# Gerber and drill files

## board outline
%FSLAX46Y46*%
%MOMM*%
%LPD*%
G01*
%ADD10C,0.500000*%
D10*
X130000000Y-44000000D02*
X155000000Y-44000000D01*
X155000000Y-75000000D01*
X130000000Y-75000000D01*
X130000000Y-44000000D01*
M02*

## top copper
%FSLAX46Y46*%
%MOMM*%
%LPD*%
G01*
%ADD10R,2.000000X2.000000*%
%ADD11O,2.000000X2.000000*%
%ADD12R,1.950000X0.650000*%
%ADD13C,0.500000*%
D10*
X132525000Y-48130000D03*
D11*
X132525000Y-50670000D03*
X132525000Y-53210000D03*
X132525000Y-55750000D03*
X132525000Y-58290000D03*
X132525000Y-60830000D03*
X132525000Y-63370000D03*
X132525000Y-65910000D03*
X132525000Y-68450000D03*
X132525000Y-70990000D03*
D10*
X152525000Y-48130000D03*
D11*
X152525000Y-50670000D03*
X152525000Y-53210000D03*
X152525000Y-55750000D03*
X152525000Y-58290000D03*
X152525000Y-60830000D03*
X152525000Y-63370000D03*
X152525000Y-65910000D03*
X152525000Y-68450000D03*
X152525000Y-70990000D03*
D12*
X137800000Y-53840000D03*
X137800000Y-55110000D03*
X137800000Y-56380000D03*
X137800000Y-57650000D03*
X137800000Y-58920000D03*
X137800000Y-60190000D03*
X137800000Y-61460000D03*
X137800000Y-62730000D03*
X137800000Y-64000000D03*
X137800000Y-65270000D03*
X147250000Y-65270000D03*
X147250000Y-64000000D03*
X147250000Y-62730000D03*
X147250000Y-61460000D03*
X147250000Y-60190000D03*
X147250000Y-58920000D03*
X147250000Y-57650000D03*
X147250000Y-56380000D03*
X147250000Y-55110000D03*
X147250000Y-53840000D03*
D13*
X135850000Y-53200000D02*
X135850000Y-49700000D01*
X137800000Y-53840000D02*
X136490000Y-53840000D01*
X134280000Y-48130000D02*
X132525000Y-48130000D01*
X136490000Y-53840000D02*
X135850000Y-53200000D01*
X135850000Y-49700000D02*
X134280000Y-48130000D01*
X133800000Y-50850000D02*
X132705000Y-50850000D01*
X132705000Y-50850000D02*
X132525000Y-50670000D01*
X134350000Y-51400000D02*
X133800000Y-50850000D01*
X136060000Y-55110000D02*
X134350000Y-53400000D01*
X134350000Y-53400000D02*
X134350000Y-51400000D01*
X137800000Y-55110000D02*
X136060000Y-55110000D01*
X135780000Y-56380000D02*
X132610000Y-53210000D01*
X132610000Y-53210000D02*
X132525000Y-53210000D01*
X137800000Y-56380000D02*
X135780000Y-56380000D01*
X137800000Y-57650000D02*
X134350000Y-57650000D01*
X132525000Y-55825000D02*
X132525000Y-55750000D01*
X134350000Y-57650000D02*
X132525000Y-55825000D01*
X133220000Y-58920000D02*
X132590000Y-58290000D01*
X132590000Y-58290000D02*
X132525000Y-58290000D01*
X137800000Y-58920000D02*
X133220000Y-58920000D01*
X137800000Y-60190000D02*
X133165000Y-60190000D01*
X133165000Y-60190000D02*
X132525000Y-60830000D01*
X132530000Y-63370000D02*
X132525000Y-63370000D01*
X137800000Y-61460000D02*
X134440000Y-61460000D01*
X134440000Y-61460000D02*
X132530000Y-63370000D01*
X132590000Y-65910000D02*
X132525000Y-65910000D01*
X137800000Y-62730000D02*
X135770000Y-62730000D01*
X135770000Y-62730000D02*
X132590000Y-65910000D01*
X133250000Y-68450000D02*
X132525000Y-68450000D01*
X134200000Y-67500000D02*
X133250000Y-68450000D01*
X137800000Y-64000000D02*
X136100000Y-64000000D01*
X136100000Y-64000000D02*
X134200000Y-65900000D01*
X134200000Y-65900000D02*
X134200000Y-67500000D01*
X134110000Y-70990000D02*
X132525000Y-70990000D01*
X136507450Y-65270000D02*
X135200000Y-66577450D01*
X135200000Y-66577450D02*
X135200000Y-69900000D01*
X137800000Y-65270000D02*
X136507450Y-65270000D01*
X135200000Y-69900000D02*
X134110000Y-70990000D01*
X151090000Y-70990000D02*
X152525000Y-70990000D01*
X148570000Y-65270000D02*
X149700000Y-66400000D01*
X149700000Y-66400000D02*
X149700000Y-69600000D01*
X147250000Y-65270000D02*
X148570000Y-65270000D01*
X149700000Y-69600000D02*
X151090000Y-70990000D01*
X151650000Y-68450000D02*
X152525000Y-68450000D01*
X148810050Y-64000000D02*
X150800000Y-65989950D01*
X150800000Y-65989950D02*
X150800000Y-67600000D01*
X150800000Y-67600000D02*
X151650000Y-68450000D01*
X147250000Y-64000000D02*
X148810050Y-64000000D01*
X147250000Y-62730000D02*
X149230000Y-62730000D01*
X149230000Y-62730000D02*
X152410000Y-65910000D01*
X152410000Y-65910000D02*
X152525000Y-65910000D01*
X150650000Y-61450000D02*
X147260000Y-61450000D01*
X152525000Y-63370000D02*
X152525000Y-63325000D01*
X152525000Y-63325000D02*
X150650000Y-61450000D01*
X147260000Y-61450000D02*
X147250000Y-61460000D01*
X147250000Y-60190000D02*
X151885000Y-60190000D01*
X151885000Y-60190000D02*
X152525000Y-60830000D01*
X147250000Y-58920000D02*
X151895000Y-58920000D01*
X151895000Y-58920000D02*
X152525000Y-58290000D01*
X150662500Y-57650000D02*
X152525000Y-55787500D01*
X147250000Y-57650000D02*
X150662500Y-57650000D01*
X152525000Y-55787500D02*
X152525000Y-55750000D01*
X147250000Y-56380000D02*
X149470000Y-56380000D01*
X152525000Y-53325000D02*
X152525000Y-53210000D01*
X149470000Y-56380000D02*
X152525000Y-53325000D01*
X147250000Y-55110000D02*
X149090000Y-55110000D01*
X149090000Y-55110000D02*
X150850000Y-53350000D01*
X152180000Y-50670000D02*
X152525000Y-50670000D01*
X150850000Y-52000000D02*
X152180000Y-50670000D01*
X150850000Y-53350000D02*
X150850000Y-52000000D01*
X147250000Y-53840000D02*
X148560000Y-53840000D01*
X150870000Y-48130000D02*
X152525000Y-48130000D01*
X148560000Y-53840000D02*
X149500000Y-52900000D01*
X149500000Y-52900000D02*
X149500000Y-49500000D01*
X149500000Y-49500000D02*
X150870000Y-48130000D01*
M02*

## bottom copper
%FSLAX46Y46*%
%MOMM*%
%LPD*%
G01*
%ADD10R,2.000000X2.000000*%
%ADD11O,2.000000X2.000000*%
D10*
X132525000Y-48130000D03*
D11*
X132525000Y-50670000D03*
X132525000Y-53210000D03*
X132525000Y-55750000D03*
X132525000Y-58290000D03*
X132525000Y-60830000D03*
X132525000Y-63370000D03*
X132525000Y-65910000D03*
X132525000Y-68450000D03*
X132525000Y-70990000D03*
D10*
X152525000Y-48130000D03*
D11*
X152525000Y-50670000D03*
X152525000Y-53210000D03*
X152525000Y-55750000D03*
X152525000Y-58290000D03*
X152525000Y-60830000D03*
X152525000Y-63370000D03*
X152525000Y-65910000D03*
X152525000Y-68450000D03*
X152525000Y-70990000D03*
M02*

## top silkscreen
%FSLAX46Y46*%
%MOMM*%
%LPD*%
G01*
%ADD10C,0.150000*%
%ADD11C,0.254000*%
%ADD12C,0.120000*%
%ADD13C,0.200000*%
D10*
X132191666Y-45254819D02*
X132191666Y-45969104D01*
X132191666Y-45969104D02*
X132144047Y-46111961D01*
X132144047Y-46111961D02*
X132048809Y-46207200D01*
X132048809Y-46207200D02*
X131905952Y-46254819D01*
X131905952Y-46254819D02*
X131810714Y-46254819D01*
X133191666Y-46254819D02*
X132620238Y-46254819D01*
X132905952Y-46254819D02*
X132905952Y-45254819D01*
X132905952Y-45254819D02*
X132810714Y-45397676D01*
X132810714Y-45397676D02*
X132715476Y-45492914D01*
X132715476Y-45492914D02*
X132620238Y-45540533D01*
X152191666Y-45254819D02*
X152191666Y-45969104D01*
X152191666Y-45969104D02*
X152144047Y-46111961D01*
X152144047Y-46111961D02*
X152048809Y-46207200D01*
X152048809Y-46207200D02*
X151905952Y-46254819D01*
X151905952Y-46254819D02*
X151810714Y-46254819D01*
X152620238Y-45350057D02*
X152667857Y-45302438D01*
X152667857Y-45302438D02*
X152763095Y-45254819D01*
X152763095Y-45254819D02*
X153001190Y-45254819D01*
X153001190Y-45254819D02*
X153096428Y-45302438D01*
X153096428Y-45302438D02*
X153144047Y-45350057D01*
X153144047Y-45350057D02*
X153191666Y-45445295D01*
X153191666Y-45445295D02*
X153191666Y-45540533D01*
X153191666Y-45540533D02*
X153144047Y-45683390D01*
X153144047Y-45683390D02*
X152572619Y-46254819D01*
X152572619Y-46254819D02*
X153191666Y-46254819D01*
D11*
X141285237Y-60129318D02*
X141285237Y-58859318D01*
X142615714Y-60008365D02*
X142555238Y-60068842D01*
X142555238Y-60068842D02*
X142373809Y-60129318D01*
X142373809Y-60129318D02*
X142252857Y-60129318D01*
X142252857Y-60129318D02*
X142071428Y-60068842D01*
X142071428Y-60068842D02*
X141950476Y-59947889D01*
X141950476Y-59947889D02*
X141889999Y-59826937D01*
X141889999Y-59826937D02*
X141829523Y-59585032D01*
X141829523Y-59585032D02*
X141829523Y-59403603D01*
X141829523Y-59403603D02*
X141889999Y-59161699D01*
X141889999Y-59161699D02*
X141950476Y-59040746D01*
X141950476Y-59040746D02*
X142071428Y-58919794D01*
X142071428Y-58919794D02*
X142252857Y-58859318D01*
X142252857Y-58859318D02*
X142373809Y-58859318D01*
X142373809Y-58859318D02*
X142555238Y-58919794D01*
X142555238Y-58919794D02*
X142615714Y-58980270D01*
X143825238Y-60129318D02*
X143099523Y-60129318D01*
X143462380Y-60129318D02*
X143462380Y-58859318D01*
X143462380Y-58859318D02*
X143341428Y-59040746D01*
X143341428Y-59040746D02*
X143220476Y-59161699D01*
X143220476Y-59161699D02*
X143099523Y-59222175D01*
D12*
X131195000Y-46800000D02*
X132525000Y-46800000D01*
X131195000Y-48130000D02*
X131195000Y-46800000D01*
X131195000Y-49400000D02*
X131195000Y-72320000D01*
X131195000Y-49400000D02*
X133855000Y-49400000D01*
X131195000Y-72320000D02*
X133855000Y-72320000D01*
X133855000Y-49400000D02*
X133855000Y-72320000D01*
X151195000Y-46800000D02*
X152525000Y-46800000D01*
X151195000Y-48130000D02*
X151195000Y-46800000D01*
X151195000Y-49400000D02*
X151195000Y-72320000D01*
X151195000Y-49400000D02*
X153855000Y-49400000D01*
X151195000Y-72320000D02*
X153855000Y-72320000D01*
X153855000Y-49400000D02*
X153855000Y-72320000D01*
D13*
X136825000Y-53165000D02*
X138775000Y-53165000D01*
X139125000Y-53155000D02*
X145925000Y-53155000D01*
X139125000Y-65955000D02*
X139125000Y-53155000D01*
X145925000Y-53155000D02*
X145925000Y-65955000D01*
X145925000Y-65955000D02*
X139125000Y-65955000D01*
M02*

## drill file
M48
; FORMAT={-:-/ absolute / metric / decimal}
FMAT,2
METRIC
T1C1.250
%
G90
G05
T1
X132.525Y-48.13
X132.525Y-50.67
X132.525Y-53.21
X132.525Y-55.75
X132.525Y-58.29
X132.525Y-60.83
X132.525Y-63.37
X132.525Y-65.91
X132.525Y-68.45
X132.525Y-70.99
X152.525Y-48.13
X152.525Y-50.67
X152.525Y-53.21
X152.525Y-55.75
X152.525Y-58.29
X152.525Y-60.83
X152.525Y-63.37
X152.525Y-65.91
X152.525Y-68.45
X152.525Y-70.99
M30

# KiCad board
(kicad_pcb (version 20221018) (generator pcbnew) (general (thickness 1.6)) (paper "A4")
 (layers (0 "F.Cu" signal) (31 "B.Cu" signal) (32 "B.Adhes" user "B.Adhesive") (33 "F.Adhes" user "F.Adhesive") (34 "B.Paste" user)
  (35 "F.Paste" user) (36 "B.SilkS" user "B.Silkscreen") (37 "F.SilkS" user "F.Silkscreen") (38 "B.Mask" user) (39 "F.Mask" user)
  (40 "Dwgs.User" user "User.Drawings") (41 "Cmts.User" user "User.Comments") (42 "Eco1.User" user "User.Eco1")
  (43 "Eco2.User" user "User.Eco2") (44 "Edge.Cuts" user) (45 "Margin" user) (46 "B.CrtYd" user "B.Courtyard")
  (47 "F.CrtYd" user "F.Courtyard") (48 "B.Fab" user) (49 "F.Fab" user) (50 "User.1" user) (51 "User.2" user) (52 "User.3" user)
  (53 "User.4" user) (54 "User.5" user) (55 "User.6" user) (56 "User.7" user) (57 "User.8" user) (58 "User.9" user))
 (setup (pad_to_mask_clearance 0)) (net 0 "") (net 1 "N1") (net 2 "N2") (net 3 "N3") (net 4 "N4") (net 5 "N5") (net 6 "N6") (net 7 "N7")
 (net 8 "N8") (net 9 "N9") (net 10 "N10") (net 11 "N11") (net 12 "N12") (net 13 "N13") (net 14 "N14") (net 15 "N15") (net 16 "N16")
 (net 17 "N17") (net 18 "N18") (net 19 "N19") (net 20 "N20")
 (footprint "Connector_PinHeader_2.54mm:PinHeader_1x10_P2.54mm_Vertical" (layer "F.Cu") (at 132.525 48.13)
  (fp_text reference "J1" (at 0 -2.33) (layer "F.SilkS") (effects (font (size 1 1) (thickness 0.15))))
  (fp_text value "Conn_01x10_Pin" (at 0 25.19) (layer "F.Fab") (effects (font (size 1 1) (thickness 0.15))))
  (fp_line (start -1.33 -1.33) (end 0 -1.33) (stroke (width 0.12) (type solid)) (layer "F.SilkS"))
  (fp_line (start -1.33 0) (end -1.33 -1.33) (stroke (width 0.12) (type solid)) (layer "F.SilkS"))
  (fp_line (start -1.33 1.27) (end -1.33 24.19) (stroke (width 0.12) (type solid)) (layer "F.SilkS"))
  (fp_line (start -1.33 1.27) (end 1.33 1.27) (stroke (width 0.12) (type solid)) (layer "F.SilkS"))
  (fp_line (start -1.33 24.19) (end 1.33 24.19) (stroke (width 0.12) (type solid)) (layer "F.SilkS"))
  (fp_line (start 1.33 1.27) (end 1.33 24.19) (stroke (width 0.12) (type solid)) (layer "F.SilkS"))
  (pad "1" thru_hole rect (at 0 0) (size 2 2) (drill 1.25) (layers "*.Cu" "*.Mask") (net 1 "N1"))
  (pad "2" thru_hole oval (at 0 2.54) (size 2 2) (drill 1.25) (layers "*.Cu" "*.Mask") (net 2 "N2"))
  (pad "3" thru_hole oval (at 0 5.08) (size 2 2) (drill 1.25) (layers "*.Cu" "*.Mask") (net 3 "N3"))
  (pad "4" thru_hole oval (at 0 7.62) (size 2 2) (drill 1.25) (layers "*.Cu" "*.Mask") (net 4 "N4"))
  (pad "5" thru_hole oval (at 0 10.16) (size 2 2) (drill 1.25) (layers "*.Cu" "*.Mask") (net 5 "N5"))
  (pad "6" thru_hole oval (at 0 12.7) (size 2 2) (drill 1.25) (layers "*.Cu" "*.Mask") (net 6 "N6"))
  (pad "7" thru_hole oval (at 0 15.24) (size 2 2) (drill 1.25) (layers "*.Cu" "*.Mask") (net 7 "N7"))
  (pad "8" thru_hole oval (at 0 17.78) (size 2 2) (drill 1.25) (layers "*.Cu" "*.Mask") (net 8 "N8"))
  (pad "9" thru_hole oval (at 0 20.32) (size 2 2) (drill 1.25) (layers "*.Cu" "*.Mask") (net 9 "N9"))
  (pad "10" thru_hole oval (at 0 22.86) (size 2 2) (drill 1.25) (layers "*.Cu" "*.Mask") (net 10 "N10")))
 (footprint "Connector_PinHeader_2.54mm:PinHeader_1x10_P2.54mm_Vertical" (layer "F.Cu") (at 152.525 48.13)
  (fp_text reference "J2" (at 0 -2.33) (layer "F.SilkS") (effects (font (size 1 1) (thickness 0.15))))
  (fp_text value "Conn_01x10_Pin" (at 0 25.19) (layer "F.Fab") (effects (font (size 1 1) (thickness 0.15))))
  (fp_line (start -1.33 -1.33) (end 0 -1.33) (stroke (width 0.12) (type solid)) (layer "F.SilkS"))
  (fp_line (start -1.33 0) (end -1.33 -1.33) (stroke (width 0.12) (type solid)) (layer "F.SilkS"))
  (fp_line (start -1.33 1.27) (end -1.33 24.19) (stroke (width 0.12) (type solid)) (layer "F.SilkS"))
  (fp_line (start -1.33 1.27) (end 1.33 1.27) (stroke (width 0.12) (type solid)) (layer "F.SilkS"))
  (fp_line (start -1.33 24.19) (end 1.33 24.19) (stroke (width 0.12) (type solid)) (layer "F.SilkS"))
  (fp_line (start 1.33 1.27) (end 1.33 24.19) (stroke (width 0.12) (type solid)) (layer "F.SilkS"))
  (pad "1" thru_hole rect (at 0 0) (size 2 2) (drill 1.25) (layers "*.Cu" "*.Mask") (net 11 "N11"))
  (pad "2" thru_hole oval (at 0 2.54) (size 2 2) (drill 1.25) (layers "*.Cu" "*.Mask") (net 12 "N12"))
  (pad "3" thru_hole oval (at 0 5.08) (size 2 2) (drill 1.25) (layers "*.Cu" "*.Mask") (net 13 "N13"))
  (pad "4" thru_hole oval (at 0 7.62) (size 2 2) (drill 1.25) (layers "*.Cu" "*.Mask") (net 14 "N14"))
  (pad "5" thru_hole oval (at 0 10.16) (size 2 2) (drill 1.25) (layers "*.Cu" "*.Mask") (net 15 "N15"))
  (pad "6" thru_hole oval (at 0 12.7) (size 2 2) (drill 1.25) (layers "*.Cu" "*.Mask") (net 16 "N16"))
  (pad "7" thru_hole oval (at 0 15.24) (size 2 2) (drill 1.25) (layers "*.Cu" "*.Mask") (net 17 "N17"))
  (pad "8" thru_hole oval (at 0 17.78) (size 2 2) (drill 1.25) (layers "*.Cu" "*.Mask") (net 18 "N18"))
  (pad "9" thru_hole oval (at 0 20.32) (size 2 2) (drill 1.25) (layers "*.Cu" "*.Mask") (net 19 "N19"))
  (pad "10" thru_hole oval (at 0 22.86) (size 2 2) (drill 1.25) (layers "*.Cu" "*.Mask") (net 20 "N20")))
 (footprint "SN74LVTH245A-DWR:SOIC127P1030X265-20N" (layer "F.Cu") (at 142.525 59.555)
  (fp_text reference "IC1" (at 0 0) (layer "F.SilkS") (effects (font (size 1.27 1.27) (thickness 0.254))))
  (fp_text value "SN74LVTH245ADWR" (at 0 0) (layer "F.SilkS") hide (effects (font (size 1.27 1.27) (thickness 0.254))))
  (fp_line (start -5.7 -6.39) (end -3.75 -6.39) (stroke (width 0.2) (type solid)) (layer "F.SilkS"))
  (fp_line (start -3.4 -6.4) (end 3.4 -6.4) (stroke (width 0.2) (type solid)) (layer "F.SilkS"))
  (fp_line (start -3.4 6.4) (end -3.4 -6.4) (stroke (width 0.2) (type solid)) (layer "F.SilkS"))
  (fp_line (start 3.4 -6.4) (end 3.4 6.4) (stroke (width 0.2) (type solid)) (layer "F.SilkS"))
  (fp_line (start 3.4 6.4) (end -3.4 6.4) (stroke (width 0.2) (type solid)) (layer "F.SilkS"))
  (pad "1" smd rect (at -4.725 -5.715 90) (size 0.65 1.95) (layers "F.Cu" "F.Paste" "F.Mask") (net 1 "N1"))
  (pad "2" smd rect (at -4.725 -4.445 90) (size 0.65 1.95) (layers "F.Cu" "F.Paste" "F.Mask") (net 2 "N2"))
  (pad "3" smd rect (at -4.725 -3.175 90) (size 0.65 1.95) (layers "F.Cu" "F.Paste" "F.Mask") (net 3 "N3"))
  (pad "4" smd rect (at -4.725 -1.905 90) (size 0.65 1.95) (layers "F.Cu" "F.Paste" "F.Mask") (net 4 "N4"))
  (pad "5" smd rect (at -4.725 -0.635 90) (size 0.65 1.95) (layers "F.Cu" "F.Paste" "F.Mask") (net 5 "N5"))
  (pad "6" smd rect (at -4.725 0.635 90) (size 0.65 1.95) (layers "F.Cu" "F.Paste" "F.Mask") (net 6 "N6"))
  (pad "7" smd rect (at -4.725 1.905 90) (size 0.65 1.95) (layers "F.Cu" "F.Paste" "F.Mask") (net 7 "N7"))
  (pad "8" smd rect (at -4.725 3.175 90) (size 0.65 1.95) (layers "F.Cu" "F.Paste" "F.Mask") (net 8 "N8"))
  (pad "9" smd rect (at -4.725 4.445 90) (size 0.65 1.95) (layers "F.Cu" "F.Paste" "F.Mask") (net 9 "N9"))
  (pad "10" smd rect (at -4.725 5.715 90) (size 0.65 1.95) (layers "F.Cu" "F.Paste" "F.Mask") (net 10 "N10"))
  (pad "11" smd rect (at 4.725 5.715 90) (size 0.65 1.95) (layers "F.Cu" "F.Paste" "F.Mask") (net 20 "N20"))
  (pad "12" smd rect (at 4.725 4.445 90) (size 0.65 1.95) (layers "F.Cu" "F.Paste" "F.Mask") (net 19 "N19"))
  (pad "13" smd rect (at 4.725 3.175 90) (size 0.65 1.95) (layers "F.Cu" "F.Paste" "F.Mask") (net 18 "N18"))
  (pad "14" smd rect (at 4.725 1.905 90) (size 0.65 1.95) (layers "F.Cu" "F.Paste" "F.Mask") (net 17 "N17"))
  (pad "15" smd rect (at 4.725 0.635 90) (size 0.65 1.95) (layers "F.Cu" "F.Paste" "F.Mask") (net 16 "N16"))
  (pad "16" smd rect (at 4.725 -0.635 90) (size 0.65 1.95) (layers "F.Cu" "F.Paste" "F.Mask") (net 15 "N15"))
  (pad "17" smd rect (at 4.725 -1.905 90) (size 0.65 1.95) (layers "F.Cu" "F.Paste" "F.Mask") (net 14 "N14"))
  (pad "18" smd rect (at 4.725 -3.175 90) (size 0.65 1.95) (layers "F.Cu" "F.Paste" "F.Mask") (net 13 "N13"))
  (pad "19" smd rect (at 4.725 -4.445 90) (size 0.65 1.95) (layers "F.Cu" "F.Paste" "F.Mask") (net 12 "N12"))
  (pad "20" smd rect (at 4.725 -5.715 90) (size 0.65 1.95) (layers "F.Cu" "F.Paste" "F.Mask") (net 11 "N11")))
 (gr_rect (start 130 44) (end 155 75) (stroke (width 0.5) (type default)) (fill none) (layer "Edge.Cuts"))
 (segment (start 135.85 53.2) (end 135.85 49.7) (width 0.5) (layer "F.Cu") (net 1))
 (segment (start 137.8 53.84) (end 136.49 53.84) (width 0.5) (layer "F.Cu") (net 1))
 (segment (start 134.28 48.13) (end 132.525 48.13) (width 0.5) (layer "F.Cu") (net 1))
 (segment (start 136.49 53.84) (end 135.85 53.2) (width 0.5) (layer "F.Cu") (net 1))
 (segment (start 135.85 49.7) (end 134.28 48.13) (width 0.5) (layer "F.Cu") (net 1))
 (segment (start 133.8 50.85) (end 132.705 50.85) (width 0.5) (layer "F.Cu") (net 2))
 (segment (start 132.705 50.85) (end 132.525 50.67) (width 0.5) (layer "F.Cu") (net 2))
 (segment (start 134.35 51.4) (end 133.8 50.85) (width 0.5) (layer "F.Cu") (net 2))
 (segment (start 136.06 55.11) (end 134.35 53.4) (width 0.5) (layer "F.Cu") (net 2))
 (segment (start 134.35 53.4) (end 134.35 51.4) (width 0.5) (layer "F.Cu") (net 2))
 (segment (start 137.8 55.11) (end 136.06 55.11) (width 0.5) (layer "F.Cu") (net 2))
 (segment (start 135.78 56.38) (end 132.61 53.21) (width 0.5) (layer "F.Cu") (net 3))
 (segment (start 132.61 53.21) (end 132.525 53.21) (width 0.5) (layer "F.Cu") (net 3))
 (segment (start 137.8 56.38) (end 135.78 56.38) (width 0.5) (layer "F.Cu") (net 3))
 (segment (start 137.8 57.65) (end 134.35 57.65) (width 0.5) (layer "F.Cu") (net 4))
 (segment (start 132.525 55.825) (end 132.525 55.75) (width 0.5) (layer "F.Cu") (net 4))
 (segment (start 134.35 57.65) (end 132.525 55.825) (width 0.5) (layer "F.Cu") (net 4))
 (segment (start 133.22 58.92) (end 132.59 58.29) (width 0.5) (layer "F.Cu") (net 5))
 (segment (start 132.59 58.29) (end 132.525 58.29) (width 0.5) (layer "F.Cu") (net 5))
 (segment (start 137.8 58.92) (end 133.22 58.92) (width 0.5) (layer "F.Cu") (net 5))
 (segment (start 137.8 60.19) (end 133.165 60.19) (width 0.5) (layer "F.Cu") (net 6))
 (segment (start 133.165 60.19) (end 132.525 60.83) (width 0.5) (layer "F.Cu") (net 6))
 (segment (start 132.53 63.37) (end 132.525 63.37) (width 0.5) (layer "F.Cu") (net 7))
 (segment (start 137.8 61.46) (end 134.44 61.46) (width 0.5) (layer "F.Cu") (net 7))
 (segment (start 134.44 61.46) (end 132.53 63.37) (width 0.5) (layer "F.Cu") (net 7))
 (segment (start 132.59 65.91) (end 132.525 65.91) (width 0.5) (layer "F.Cu") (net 8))
 (segment (start 137.8 62.73) (end 135.77 62.73) (width 0.5) (layer "F.Cu") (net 8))
 (segment (start 135.77 62.73) (end 132.59 65.91) (width 0.5) (layer "F.Cu") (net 8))
 (segment (start 133.25 68.45) (end 132.525 68.45) (width 0.5) (layer "F.Cu") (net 9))
 (segment (start 134.2 67.5) (end 133.25 68.45) (width 0.5) (layer "F.Cu") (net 9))
 (segment (start 137.8 64) (end 136.1 64) (width 0.5) (layer "F.Cu") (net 9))
 (segment (start 136.1 64) (end 134.2 65.9) (width 0.5) (layer "F.Cu") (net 9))
 (segment (start 134.2 65.9) (end 134.2 67.5) (width 0.5) (layer "F.Cu") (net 9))
 (segment (start 134.11 70.99) (end 132.525 70.99) (width 0.5) (layer "F.Cu") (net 10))
 (segment (start 136.50745 65.27) (end 135.2 66.57745) (width 0.5) (layer "F.Cu") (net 10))
 (segment (start 135.2 66.57745) (end 135.2 69.9) (width 0.5) (layer "F.Cu") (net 10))
 (segment (start 137.8 65.27) (end 136.50745 65.27) (width 0.5) (layer "F.Cu") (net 10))
 (segment (start 135.2 69.9) (end 134.11 70.99) (width 0.5) (layer "F.Cu") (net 10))
 (segment (start 151.09 70.99) (end 152.525 70.99) (width 0.5) (layer "F.Cu") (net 20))
 (segment (start 148.57 65.27) (end 149.7 66.4) (width 0.5) (layer "F.Cu") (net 20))
 (segment (start 149.7 66.4) (end 149.7 69.6) (width 0.5) (layer "F.Cu") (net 20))
 (segment (start 147.25 65.27) (end 148.57 65.27) (width 0.5) (layer "F.Cu") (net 20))
 (segment (start 149.7 69.6) (end 151.09 70.99) (width 0.5) (layer "F.Cu") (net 20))
 (segment (start 151.65 68.45) (end 152.525 68.45) (width 0.5) (layer "F.Cu") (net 19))
 (segment (start 148.81005 64) (end 150.8 65.98995) (width 0.5) (layer "F.Cu") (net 19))
 (segment (start 150.8 65.98995) (end 150.8 67.6) (width 0.5) (layer "F.Cu") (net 19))
 (segment (start 150.8 67.6) (end 151.65 68.45) (width 0.5) (layer "F.Cu") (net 19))
 (segment (start 147.25 64) (end 148.81005 64) (width 0.5) (layer "F.Cu") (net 19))
 (segment (start 147.25 62.73) (end 149.23 62.73) (width 0.5) (layer "F.Cu") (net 18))
 (segment (start 149.23 62.73) (end 152.41 65.91) (width 0.5) (layer "F.Cu") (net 18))
 (segment (start 152.41 65.91) (end 152.525 65.91) (width 0.5) (layer "F.Cu") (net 18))
 (segment (start 150.65 61.45) (end 147.26 61.45) (width 0.5) (layer "F.Cu") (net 17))
 (segment (start 152.525 63.37) (end 152.525 63.325) (width 0.5) (layer "F.Cu") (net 17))
 (segment (start 152.525 63.325) (end 150.65 61.45) (width 0.5) (layer "F.Cu") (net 17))
 (segment (start 147.26 61.45) (end 147.25 61.46) (width 0.5) (layer "F.Cu") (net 17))
 (segment (start 147.25 60.19) (end 151.885 60.19) (width 0.5) (layer "F.Cu") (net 16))
 (segment (start 151.885 60.19) (end 152.525 60.83) (width 0.5) (layer "F.Cu") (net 16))
 (segment (start 147.25 58.92) (end 151.895 58.92) (width 0.5) (layer "F.Cu") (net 15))
 (segment (start 151.895 58.92) (end 152.525 58.29) (width 0.5) (layer "F.Cu") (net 15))
 (segment (start 150.6625 57.65) (end 152.525 55.7875) (width 0.5) (layer "F.Cu") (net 14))
 (segment (start 147.25 57.65) (end 150.6625 57.65) (width 0.5) (layer "F.Cu") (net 14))
 (segment (start 152.525 55.7875) (end 152.525 55.75) (width 0.5) (layer "F.Cu") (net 14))
 (segment (start 147.25 56.38) (end 149.47 56.38) (width 0.5) (layer "F.Cu") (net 13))
 (segment (start 152.525 53.325) (end 152.525 53.21) (width 0.5) (layer "F.Cu") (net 13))
 (segment (start 149.47 56.38) (end 152.525 53.325) (width 0.5) (layer "F.Cu") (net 13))
 (segment (start 147.25 55.11) (end 149.09 55.11) (width 0.5) (layer "F.Cu") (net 12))
 (segment (start 149.09 55.11) (end 150.85 53.35) (width 0.5) (layer "F.Cu") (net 12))
 (segment (start 152.18 50.67) (end 152.525 50.67) (width 0.5) (layer "F.Cu") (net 12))
 (segment (start 150.85 52) (end 152.18 50.67) (width 0.5) (layer "F.Cu") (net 12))
 (segment (start 150.85 53.35) (end 150.85 52) (width 0.5) (layer "F.Cu") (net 12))
 (segment (start 147.25 53.84) (end 148.56 53.84) (width 0.5) (layer "F.Cu") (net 11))
 (segment (start 150.87 48.13) (end 152.525 48.13) (width 0.5) (layer "F.Cu") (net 11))
 (segment (start 148.56 53.84) (end 149.5 52.9) (width 0.5) (layer "F.Cu") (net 11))
 (segment (start 149.5 52.9) (end 149.5 49.5) (width 0.5) (layer "F.Cu") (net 11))
 (segment (start 149.5 49.5) (end 150.87 48.13) (width 0.5) (layer "F.Cu") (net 11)))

